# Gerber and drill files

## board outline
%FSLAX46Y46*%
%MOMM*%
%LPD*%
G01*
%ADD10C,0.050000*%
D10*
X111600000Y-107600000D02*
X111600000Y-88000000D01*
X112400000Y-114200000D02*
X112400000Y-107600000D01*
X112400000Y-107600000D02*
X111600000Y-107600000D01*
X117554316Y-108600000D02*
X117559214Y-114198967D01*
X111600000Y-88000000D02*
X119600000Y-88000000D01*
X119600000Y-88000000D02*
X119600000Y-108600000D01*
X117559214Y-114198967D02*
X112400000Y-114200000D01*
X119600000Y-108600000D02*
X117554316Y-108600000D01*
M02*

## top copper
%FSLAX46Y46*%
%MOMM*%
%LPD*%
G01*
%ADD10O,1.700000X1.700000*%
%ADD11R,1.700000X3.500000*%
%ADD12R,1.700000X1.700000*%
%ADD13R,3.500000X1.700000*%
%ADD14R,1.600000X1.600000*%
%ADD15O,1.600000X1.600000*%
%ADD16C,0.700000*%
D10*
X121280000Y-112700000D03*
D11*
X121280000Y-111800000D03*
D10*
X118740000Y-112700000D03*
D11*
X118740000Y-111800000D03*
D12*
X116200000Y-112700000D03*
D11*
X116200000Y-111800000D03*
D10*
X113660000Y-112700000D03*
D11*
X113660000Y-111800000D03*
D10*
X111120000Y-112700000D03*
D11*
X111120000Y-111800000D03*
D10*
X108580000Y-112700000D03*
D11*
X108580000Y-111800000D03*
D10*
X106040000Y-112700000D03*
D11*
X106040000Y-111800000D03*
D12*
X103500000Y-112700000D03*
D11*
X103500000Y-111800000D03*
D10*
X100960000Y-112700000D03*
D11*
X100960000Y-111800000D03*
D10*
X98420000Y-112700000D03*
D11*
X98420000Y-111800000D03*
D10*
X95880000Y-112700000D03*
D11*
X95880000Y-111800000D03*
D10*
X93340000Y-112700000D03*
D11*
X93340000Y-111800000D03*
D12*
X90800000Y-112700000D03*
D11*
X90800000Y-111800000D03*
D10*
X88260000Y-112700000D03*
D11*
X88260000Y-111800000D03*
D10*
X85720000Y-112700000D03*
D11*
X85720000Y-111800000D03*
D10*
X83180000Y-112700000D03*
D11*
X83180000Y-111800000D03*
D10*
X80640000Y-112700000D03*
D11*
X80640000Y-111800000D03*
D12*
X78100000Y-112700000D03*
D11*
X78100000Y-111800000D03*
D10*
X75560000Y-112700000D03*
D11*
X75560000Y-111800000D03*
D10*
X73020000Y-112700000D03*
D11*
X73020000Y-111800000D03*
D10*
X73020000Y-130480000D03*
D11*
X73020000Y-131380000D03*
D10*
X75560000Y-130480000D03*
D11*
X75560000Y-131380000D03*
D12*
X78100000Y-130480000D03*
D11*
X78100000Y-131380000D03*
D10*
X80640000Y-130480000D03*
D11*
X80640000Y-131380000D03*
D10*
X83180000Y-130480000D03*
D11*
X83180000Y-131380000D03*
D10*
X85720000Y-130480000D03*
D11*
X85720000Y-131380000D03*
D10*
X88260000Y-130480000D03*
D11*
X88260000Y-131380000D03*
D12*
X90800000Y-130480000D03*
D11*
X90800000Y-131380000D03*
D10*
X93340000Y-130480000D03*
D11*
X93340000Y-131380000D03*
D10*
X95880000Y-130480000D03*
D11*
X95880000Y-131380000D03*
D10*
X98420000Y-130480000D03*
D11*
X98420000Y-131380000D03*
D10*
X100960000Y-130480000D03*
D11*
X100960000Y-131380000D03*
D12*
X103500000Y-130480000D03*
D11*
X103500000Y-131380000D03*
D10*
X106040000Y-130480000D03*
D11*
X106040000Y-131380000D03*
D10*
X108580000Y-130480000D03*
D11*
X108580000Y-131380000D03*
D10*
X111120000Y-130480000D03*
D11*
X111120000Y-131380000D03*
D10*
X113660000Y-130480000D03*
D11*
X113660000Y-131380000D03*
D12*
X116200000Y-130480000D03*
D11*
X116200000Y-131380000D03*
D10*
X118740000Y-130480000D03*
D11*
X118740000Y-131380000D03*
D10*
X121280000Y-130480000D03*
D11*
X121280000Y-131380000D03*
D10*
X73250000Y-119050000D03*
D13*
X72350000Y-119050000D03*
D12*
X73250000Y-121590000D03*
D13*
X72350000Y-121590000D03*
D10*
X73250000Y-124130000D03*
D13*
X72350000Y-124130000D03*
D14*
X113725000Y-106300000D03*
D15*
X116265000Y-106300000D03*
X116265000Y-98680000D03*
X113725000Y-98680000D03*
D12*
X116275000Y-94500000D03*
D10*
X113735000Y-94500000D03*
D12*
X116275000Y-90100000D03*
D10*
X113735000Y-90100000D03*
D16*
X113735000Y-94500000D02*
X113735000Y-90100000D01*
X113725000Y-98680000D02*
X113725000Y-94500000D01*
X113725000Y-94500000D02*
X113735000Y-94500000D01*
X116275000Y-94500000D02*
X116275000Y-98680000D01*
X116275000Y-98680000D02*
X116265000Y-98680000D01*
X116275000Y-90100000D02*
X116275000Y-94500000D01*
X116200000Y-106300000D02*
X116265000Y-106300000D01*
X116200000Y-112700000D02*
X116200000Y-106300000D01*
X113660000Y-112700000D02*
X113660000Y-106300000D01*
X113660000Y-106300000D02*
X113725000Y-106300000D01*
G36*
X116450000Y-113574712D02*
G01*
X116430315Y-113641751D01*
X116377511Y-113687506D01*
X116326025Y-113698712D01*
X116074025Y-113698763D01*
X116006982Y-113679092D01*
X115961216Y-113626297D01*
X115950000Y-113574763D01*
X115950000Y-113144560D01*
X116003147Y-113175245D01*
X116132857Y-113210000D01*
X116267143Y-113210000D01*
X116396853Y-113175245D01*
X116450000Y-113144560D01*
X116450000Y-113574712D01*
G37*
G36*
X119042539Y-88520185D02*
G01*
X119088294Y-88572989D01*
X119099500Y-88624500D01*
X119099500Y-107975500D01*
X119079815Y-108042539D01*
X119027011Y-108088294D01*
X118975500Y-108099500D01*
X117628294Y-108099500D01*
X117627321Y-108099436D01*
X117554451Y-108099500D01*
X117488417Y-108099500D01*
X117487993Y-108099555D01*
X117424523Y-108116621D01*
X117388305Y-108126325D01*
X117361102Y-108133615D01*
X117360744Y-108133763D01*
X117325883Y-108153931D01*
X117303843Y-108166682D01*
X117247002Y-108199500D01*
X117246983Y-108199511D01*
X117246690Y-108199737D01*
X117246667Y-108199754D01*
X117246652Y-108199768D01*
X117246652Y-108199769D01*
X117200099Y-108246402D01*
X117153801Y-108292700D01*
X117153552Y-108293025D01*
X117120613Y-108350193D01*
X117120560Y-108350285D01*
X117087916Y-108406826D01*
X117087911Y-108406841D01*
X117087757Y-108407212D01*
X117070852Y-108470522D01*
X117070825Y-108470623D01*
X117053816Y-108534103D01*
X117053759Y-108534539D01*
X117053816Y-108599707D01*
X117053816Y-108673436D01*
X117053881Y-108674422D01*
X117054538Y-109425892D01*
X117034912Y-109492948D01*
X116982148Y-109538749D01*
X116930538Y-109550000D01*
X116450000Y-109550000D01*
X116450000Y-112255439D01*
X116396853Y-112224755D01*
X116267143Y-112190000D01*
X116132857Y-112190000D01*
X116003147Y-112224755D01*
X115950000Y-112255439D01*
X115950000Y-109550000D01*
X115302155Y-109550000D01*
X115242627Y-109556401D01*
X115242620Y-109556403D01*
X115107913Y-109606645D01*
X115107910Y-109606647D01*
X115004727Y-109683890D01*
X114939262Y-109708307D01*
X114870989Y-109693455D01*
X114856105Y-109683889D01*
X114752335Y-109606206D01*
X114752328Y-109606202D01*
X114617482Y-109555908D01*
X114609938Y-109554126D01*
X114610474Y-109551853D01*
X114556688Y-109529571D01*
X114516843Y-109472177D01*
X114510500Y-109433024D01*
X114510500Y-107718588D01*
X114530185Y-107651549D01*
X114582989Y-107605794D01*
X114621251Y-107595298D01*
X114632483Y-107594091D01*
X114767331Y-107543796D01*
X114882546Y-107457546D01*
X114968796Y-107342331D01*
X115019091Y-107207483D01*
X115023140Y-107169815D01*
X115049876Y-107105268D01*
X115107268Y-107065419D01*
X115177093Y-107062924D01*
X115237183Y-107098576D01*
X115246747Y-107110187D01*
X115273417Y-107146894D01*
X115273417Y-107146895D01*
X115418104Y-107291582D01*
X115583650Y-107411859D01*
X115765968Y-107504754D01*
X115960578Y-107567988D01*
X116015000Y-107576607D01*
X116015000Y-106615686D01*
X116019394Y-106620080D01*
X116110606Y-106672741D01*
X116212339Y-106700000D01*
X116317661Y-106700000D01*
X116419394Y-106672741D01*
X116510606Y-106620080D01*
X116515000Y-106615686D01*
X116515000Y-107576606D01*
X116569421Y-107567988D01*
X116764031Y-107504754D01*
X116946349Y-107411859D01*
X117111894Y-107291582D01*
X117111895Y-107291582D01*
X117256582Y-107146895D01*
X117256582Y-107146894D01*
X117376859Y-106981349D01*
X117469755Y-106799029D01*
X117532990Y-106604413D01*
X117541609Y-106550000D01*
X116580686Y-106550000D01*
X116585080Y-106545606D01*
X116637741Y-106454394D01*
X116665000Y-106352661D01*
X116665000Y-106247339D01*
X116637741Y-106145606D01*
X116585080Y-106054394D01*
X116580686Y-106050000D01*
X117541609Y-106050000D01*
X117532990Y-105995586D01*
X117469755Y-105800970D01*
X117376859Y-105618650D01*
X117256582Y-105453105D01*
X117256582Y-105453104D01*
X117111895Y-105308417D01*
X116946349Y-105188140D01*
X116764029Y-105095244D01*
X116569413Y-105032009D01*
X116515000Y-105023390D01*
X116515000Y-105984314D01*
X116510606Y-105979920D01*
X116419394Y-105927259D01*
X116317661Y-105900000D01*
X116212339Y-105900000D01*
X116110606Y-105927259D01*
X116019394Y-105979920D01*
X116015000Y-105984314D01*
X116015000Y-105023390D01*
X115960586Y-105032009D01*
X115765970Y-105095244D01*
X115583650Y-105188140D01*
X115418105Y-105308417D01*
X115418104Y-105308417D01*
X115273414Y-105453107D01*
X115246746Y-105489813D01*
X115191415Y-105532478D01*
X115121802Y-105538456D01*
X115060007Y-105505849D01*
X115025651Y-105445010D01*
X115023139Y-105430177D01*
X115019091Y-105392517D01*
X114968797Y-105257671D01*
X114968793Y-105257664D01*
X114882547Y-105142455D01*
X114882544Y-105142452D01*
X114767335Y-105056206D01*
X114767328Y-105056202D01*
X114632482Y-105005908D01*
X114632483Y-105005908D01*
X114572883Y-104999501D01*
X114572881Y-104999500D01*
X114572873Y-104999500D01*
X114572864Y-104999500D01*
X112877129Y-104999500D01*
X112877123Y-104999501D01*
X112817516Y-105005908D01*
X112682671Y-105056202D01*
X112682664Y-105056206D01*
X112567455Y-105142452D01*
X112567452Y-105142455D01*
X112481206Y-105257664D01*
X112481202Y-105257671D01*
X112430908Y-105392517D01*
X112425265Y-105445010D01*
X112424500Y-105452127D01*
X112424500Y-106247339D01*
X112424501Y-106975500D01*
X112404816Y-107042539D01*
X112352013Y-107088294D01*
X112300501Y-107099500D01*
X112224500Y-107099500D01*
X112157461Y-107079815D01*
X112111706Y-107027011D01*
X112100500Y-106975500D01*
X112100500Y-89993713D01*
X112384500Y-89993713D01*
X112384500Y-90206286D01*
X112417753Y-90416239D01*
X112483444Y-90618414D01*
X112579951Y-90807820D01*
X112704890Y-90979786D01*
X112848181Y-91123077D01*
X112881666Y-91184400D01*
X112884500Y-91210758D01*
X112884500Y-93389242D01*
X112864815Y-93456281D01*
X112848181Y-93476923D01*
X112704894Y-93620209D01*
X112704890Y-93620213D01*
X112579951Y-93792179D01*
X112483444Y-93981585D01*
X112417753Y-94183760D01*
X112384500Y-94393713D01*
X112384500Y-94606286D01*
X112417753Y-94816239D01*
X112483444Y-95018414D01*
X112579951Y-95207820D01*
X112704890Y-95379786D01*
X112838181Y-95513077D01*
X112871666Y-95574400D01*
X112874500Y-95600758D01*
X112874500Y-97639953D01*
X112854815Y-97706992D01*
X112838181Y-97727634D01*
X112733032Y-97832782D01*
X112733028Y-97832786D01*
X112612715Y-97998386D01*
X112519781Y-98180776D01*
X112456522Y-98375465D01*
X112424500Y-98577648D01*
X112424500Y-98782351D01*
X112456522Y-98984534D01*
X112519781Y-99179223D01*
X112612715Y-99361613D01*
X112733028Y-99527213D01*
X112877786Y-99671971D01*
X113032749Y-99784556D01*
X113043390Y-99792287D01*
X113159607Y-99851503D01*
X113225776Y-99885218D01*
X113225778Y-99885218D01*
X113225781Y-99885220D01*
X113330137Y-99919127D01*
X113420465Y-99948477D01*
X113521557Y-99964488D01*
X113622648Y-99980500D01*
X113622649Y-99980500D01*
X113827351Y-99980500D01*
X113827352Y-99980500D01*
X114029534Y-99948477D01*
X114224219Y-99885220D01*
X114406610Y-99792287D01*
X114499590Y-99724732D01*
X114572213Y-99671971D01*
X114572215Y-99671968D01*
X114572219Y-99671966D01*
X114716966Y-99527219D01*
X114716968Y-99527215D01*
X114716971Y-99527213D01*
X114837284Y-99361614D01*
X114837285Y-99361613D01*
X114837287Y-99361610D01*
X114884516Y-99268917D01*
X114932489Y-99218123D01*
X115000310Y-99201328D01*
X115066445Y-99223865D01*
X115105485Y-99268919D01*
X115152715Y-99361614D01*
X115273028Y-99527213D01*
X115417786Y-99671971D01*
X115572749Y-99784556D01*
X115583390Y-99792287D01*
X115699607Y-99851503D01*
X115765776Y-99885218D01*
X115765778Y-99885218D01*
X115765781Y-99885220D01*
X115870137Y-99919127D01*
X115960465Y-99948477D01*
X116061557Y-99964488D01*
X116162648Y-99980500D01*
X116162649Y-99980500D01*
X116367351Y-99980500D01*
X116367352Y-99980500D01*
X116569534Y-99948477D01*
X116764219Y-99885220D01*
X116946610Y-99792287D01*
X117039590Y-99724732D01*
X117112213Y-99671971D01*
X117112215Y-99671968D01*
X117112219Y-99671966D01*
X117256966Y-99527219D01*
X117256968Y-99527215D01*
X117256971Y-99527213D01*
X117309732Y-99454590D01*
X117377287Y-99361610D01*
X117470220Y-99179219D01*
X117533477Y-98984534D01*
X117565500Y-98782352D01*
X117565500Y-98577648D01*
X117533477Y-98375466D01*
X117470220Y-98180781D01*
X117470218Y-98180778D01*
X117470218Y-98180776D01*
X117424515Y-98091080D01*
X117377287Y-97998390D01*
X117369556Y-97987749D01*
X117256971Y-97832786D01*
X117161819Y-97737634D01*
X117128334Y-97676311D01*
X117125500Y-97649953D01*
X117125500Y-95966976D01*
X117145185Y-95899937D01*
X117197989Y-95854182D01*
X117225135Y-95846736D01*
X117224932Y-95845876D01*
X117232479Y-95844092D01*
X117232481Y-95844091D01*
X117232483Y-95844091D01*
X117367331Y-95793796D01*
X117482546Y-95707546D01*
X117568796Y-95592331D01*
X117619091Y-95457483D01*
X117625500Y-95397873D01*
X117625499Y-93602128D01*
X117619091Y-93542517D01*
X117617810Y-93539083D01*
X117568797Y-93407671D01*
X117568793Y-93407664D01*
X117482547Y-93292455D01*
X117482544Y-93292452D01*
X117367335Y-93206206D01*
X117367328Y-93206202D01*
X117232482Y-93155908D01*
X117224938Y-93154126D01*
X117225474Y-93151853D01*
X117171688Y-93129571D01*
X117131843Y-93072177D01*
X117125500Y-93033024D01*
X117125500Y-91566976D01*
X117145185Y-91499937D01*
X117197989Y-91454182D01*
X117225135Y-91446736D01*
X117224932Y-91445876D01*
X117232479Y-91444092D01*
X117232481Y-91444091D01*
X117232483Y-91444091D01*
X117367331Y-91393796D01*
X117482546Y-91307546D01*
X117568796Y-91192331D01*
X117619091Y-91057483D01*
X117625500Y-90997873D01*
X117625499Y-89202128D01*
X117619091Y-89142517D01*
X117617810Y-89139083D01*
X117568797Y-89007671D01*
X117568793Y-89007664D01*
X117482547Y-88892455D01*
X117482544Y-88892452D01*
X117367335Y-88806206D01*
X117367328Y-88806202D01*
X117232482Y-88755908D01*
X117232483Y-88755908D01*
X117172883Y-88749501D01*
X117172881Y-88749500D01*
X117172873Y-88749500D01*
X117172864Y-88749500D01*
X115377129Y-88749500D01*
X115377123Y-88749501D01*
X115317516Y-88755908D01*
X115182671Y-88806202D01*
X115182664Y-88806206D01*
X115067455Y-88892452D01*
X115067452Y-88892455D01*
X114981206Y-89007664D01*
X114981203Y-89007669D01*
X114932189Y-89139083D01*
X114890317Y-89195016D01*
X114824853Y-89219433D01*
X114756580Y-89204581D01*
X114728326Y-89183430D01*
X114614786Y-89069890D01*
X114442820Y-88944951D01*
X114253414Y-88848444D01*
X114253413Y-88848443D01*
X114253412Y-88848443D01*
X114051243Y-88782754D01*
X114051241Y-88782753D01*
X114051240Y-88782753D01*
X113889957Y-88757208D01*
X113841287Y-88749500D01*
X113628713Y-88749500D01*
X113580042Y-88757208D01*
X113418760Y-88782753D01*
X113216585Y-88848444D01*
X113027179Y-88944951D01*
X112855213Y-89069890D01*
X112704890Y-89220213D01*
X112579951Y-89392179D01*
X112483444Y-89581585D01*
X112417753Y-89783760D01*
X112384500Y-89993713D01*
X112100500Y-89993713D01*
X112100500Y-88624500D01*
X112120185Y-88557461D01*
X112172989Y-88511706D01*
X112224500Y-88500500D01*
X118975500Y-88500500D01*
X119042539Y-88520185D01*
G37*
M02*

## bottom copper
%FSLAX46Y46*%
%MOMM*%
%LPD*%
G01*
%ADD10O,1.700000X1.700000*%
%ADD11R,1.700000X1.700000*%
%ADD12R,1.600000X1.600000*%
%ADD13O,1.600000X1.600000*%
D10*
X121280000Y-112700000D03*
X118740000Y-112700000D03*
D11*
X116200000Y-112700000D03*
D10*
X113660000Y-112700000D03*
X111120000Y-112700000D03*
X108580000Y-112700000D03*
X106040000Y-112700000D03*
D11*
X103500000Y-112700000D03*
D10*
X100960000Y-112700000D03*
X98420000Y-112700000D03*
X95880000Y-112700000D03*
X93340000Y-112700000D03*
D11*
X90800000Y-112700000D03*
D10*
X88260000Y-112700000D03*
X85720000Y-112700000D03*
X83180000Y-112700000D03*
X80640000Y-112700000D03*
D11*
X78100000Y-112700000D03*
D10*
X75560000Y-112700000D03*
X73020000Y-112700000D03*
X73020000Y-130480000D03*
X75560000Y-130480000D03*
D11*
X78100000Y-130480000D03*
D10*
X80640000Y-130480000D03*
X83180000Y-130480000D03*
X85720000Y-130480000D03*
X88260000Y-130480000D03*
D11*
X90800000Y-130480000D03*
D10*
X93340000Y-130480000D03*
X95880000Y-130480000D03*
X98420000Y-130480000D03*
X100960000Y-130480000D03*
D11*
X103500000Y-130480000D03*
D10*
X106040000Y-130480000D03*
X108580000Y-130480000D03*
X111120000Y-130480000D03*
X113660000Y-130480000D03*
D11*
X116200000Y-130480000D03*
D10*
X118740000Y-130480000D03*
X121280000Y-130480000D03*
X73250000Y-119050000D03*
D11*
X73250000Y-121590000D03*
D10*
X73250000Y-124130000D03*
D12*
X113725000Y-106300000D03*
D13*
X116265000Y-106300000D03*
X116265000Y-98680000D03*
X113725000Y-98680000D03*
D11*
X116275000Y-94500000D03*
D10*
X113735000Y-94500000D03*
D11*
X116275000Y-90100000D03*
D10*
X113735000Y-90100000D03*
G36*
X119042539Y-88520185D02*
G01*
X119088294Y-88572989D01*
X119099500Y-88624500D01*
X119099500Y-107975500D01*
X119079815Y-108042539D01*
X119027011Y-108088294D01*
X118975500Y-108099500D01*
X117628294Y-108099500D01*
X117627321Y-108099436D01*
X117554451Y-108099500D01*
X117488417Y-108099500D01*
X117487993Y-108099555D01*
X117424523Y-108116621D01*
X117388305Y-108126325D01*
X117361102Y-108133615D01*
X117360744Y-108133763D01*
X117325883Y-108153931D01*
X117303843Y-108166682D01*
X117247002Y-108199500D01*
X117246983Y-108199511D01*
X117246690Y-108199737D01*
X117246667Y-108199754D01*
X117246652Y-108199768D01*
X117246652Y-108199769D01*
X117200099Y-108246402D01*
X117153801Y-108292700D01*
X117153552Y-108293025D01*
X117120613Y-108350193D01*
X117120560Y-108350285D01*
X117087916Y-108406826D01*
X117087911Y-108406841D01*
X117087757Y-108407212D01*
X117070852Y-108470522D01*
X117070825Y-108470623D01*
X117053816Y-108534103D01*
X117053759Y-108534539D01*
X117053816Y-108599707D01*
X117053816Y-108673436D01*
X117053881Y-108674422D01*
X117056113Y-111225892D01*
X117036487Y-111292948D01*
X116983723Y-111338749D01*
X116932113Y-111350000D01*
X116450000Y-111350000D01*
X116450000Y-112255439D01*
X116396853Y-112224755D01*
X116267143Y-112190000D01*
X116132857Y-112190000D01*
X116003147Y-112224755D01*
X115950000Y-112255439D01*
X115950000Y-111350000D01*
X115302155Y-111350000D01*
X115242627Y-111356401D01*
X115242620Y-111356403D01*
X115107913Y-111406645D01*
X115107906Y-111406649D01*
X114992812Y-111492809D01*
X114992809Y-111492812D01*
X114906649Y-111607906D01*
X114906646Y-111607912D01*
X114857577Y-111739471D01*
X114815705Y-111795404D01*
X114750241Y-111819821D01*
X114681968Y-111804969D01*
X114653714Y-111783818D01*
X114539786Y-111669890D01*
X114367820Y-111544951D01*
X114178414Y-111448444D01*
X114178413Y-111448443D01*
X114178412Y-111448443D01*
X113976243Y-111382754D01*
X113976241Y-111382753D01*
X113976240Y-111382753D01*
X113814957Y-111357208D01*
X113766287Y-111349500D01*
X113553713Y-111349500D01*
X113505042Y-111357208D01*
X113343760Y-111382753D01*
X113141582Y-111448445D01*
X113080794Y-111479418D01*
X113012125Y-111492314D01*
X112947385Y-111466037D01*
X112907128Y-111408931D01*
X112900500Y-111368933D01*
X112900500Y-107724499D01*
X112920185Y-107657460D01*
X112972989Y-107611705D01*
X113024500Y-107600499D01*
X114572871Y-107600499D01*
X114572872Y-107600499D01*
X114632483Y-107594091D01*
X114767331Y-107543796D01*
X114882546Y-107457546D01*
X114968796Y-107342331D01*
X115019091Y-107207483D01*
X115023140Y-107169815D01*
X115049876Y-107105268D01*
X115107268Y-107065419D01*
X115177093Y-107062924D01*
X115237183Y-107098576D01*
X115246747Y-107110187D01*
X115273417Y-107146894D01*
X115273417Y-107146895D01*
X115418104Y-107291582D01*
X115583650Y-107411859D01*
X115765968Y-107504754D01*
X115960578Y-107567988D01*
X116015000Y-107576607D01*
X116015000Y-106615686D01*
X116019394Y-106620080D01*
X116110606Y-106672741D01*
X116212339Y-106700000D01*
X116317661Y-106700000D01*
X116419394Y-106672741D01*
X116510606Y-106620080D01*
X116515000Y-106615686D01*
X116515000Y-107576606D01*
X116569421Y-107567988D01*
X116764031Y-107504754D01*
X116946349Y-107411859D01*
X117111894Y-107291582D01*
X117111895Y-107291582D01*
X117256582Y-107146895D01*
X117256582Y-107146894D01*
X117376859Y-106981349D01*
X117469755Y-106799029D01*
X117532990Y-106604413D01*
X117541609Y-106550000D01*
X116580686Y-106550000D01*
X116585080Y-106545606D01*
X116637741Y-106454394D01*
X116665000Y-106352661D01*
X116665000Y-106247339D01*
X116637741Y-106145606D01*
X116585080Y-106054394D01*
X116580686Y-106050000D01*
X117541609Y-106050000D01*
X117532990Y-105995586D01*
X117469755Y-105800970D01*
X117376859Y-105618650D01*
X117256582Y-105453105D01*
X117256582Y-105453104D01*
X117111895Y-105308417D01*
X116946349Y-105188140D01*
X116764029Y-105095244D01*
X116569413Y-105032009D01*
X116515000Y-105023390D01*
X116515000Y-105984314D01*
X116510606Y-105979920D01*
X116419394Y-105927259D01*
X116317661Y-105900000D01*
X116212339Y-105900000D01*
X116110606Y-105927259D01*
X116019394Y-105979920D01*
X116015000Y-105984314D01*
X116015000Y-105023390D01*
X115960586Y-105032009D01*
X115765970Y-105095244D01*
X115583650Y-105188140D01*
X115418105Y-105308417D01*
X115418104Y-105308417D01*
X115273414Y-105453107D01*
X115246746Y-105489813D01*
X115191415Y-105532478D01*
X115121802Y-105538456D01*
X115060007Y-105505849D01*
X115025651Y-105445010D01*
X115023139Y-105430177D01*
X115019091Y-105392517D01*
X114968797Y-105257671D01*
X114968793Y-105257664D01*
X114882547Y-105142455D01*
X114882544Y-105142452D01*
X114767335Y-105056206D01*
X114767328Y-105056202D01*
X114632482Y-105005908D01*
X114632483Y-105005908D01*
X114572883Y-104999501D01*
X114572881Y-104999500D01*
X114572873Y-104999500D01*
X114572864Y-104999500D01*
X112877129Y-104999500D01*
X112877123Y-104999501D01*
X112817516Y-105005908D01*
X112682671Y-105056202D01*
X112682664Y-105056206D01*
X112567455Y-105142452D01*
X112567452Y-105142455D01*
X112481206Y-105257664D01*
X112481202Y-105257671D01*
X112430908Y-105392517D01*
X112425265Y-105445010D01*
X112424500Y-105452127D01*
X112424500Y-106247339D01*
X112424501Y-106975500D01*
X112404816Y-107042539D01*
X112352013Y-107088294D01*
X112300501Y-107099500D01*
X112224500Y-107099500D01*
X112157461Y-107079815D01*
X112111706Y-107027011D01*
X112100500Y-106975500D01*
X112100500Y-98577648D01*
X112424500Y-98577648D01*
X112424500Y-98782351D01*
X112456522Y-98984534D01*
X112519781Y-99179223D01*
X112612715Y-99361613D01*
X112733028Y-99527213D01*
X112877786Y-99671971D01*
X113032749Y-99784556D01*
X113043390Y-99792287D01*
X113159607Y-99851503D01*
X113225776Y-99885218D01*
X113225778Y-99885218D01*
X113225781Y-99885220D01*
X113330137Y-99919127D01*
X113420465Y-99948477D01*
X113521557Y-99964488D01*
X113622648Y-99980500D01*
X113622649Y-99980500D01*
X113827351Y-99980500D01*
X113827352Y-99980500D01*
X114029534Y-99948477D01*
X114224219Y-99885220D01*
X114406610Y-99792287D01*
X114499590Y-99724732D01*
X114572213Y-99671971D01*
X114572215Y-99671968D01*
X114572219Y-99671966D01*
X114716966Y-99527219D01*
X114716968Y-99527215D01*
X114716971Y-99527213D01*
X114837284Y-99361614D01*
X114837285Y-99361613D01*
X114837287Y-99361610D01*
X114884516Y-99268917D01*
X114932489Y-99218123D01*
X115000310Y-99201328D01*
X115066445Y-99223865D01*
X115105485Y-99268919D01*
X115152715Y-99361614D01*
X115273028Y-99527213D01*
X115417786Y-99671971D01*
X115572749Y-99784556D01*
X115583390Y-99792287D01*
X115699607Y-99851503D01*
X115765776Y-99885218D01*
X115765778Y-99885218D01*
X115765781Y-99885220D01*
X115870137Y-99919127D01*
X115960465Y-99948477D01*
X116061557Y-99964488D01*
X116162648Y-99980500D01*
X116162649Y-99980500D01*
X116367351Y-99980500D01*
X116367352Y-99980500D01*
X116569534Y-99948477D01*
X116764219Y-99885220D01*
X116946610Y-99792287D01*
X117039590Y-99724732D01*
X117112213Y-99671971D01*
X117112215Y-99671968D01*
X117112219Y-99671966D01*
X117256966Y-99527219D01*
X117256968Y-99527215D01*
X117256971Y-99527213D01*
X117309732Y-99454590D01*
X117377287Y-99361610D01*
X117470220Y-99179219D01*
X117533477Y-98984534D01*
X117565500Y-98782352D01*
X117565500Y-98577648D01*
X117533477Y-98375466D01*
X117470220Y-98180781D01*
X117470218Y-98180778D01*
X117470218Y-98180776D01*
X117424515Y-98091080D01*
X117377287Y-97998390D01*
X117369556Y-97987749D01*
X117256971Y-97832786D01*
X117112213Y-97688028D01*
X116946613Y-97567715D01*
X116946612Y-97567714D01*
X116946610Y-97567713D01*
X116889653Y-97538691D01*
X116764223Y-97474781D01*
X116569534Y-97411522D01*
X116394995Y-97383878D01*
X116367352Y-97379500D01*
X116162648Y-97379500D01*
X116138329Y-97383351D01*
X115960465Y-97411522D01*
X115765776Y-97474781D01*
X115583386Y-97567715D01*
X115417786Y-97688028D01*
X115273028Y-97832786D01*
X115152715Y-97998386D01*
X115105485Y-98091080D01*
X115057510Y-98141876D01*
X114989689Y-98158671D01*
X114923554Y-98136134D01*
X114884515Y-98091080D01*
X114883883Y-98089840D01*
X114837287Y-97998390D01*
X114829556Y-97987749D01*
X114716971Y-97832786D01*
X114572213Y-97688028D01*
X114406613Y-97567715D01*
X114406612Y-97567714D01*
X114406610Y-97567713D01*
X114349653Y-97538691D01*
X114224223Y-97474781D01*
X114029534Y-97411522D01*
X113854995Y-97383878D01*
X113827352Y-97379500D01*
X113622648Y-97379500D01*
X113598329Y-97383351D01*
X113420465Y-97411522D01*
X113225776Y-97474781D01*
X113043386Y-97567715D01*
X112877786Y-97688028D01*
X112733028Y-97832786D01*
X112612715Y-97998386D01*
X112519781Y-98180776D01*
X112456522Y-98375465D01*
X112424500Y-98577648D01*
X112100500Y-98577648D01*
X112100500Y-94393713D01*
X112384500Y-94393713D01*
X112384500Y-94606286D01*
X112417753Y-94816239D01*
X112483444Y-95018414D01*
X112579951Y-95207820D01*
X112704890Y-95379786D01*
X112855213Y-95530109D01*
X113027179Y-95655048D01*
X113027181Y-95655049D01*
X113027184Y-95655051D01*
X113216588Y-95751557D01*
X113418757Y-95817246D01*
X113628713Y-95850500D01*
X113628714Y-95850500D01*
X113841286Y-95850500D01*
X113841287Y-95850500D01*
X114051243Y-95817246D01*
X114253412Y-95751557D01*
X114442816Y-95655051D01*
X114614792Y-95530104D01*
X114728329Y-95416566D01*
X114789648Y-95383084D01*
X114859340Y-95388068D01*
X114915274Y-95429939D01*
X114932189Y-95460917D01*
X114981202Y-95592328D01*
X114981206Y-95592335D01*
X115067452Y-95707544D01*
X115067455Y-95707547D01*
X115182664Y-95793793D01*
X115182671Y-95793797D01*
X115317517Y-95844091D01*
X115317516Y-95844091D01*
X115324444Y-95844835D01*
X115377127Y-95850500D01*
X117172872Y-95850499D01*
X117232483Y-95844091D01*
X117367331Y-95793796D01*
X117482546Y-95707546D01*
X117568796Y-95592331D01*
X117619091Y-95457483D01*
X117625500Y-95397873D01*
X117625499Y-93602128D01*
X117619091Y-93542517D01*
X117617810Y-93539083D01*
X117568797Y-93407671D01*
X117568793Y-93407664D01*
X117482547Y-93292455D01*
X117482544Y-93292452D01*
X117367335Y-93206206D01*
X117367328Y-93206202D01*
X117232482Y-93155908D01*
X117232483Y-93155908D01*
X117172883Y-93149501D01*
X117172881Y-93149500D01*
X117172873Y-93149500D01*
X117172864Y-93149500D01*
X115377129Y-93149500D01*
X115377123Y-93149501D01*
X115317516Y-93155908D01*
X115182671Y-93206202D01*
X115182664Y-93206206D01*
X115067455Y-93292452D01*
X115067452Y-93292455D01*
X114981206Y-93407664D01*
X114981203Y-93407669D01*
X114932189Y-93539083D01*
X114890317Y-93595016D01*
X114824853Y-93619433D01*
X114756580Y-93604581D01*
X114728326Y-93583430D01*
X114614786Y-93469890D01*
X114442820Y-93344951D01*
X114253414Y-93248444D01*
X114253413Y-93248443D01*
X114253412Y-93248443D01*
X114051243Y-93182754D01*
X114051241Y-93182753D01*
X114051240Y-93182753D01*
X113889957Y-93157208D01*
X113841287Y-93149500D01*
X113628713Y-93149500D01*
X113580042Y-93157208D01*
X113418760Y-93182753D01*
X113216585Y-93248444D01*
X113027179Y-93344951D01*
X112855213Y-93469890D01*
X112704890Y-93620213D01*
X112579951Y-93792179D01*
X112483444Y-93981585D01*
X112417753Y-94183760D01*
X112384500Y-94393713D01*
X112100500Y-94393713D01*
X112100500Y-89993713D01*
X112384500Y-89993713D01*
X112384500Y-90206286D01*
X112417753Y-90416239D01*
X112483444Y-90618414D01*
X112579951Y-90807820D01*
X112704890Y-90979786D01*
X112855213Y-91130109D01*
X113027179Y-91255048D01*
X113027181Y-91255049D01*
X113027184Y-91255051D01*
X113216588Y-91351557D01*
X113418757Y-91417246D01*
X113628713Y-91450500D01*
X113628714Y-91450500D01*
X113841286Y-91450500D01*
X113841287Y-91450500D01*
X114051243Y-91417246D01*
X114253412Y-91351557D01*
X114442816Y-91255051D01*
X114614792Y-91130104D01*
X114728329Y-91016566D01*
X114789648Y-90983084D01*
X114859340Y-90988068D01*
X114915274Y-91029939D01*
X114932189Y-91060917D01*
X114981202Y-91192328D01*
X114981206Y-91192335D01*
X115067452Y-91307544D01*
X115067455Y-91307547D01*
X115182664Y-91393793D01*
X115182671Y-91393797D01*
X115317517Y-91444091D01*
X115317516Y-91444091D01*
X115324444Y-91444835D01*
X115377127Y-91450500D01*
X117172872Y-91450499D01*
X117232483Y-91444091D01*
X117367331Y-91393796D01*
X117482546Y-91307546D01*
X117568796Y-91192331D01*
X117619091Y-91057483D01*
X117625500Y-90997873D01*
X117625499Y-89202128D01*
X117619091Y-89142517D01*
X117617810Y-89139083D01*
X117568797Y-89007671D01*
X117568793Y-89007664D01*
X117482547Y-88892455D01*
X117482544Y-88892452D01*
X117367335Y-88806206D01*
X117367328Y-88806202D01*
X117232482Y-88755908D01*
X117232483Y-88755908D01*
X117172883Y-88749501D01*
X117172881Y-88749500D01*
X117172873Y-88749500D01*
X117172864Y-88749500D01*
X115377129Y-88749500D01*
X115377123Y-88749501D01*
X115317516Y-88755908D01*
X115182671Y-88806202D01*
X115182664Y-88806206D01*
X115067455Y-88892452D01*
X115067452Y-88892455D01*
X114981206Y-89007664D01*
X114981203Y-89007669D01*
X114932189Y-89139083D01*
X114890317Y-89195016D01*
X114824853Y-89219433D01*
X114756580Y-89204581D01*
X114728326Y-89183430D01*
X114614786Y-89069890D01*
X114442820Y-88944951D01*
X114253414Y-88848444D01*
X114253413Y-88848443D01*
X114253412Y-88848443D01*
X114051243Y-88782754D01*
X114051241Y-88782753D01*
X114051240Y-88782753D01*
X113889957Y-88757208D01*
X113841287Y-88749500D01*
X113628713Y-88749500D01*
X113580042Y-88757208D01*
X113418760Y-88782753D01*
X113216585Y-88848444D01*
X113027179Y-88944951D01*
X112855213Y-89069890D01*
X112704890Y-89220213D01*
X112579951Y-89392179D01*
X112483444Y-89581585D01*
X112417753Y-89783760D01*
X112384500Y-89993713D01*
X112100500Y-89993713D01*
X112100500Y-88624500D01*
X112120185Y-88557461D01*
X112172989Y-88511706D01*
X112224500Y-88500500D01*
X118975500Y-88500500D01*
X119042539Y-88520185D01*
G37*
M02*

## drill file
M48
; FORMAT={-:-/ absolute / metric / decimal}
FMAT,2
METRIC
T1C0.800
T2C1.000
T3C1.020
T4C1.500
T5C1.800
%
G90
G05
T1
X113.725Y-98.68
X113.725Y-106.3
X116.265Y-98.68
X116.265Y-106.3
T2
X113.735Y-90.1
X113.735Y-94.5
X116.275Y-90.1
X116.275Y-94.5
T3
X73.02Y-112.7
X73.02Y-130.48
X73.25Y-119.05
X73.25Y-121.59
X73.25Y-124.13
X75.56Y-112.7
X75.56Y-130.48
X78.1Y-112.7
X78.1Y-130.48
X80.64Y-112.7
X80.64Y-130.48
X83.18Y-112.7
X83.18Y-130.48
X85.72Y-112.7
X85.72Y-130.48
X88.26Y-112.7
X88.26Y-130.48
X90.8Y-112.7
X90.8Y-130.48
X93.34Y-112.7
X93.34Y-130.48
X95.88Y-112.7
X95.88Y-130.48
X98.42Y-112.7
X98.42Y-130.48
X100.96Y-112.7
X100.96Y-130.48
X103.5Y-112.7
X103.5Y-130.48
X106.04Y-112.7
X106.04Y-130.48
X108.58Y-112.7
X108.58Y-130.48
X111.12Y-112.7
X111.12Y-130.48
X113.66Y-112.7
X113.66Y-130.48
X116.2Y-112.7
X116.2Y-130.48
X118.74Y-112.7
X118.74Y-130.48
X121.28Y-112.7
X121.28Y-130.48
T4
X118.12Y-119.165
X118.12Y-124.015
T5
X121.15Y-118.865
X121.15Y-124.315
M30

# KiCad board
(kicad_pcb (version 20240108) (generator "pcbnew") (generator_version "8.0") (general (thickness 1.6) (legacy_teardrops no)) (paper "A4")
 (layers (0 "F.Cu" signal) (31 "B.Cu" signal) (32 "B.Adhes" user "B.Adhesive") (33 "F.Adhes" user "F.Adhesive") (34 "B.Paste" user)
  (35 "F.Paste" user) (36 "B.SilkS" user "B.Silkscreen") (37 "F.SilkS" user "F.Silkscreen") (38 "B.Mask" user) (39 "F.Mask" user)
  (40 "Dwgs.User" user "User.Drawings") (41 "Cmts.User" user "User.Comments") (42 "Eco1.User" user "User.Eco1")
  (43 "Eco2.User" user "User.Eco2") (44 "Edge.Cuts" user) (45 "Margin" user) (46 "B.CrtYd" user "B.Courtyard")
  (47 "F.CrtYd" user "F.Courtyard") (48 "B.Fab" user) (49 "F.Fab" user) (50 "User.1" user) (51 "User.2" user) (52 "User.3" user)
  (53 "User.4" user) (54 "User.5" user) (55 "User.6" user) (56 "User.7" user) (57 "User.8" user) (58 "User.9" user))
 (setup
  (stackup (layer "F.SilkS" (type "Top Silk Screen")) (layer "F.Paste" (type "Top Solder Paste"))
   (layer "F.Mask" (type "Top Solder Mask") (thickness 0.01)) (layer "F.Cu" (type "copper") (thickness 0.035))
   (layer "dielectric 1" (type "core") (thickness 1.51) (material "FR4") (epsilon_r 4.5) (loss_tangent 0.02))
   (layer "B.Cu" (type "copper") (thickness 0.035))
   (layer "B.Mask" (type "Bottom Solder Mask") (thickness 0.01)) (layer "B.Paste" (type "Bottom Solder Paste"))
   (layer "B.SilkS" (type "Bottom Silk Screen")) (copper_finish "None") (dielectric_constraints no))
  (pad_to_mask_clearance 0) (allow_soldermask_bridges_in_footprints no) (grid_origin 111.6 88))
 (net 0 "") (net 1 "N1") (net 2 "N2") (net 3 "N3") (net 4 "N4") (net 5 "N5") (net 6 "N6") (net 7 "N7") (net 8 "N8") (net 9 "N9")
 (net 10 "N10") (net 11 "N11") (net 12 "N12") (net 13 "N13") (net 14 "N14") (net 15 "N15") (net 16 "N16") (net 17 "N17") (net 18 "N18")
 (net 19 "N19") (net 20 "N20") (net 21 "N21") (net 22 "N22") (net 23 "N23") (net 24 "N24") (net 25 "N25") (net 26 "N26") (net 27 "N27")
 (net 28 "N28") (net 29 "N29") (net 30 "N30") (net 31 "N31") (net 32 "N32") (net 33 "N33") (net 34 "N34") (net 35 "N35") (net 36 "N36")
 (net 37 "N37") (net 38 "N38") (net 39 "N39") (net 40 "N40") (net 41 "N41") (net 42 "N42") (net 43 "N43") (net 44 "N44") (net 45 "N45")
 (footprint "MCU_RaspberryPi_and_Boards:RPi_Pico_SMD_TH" (layer "F.Cu") (at 97.15 121.59 -90)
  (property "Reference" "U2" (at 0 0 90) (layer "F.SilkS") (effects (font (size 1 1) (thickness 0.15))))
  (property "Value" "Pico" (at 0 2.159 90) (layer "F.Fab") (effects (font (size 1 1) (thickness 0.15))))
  (pad "" np_thru_hole oval (at -2.725 -24 270) (size 1.8 1.8) (drill 1.8) (layers "*.Cu" "*.Mask"))
  (pad "" np_thru_hole oval (at -2.425 -20.97 270) (size 1.5 1.5) (drill 1.5) (layers "*.Cu" "*.Mask"))
  (pad "" np_thru_hole oval (at 2.425 -20.97 270) (size 1.5 1.5) (drill 1.5) (layers "*.Cu" "*.Mask"))
  (pad "" np_thru_hole oval (at 2.725 -24 270) (size 1.8 1.8) (drill 1.8) (layers "*.Cu" "*.Mask"))
  (pad "1" thru_hole oval (at -8.89 -24.13 270) (size 1.7 1.7) (drill 1.02) (layers "*.Cu" "*.Mask") (remove_unused_layers no) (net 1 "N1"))
  (pad "1" smd rect (at -8.89 -24.13 270) (size 3.5 1.7) (drill (offset -0.9 0)) (layers "F.Cu" "F.Mask") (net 1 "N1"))
  (pad "2" thru_hole oval (at -8.89 -21.59 270) (size 1.7 1.7) (drill 1.02) (layers "*.Cu" "*.Mask") (remove_unused_layers no) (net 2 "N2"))
  (pad "2" smd rect (at -8.89 -21.59 270) (size 3.5 1.7) (drill (offset -0.9 0)) (layers "F.Cu" "F.Mask") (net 2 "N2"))
  (pad "3" thru_hole rect (at -8.89 -19.05 270) (size 1.7 1.7) (drill 1.02) (layers "*.Cu" "*.Mask") (remove_unused_layers no) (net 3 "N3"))
  (pad "3" smd rect (at -8.89 -19.05 270) (size 3.5 1.7) (drill (offset -0.9 0)) (layers "F.Cu" "F.Mask") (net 3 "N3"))
  (pad "4" thru_hole oval (at -8.89 -16.51 270) (size 1.7 1.7) (drill 1.02) (layers "*.Cu" "*.Mask") (remove_unused_layers no) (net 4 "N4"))
  (pad "4" smd rect (at -8.89 -16.51 270) (size 3.5 1.7) (drill (offset -0.9 0)) (layers "F.Cu" "F.Mask") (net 4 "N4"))
  (pad "5" thru_hole oval (at -8.89 -13.97 270) (size 1.7 1.7) (drill 1.02) (layers "*.Cu" "*.Mask") (remove_unused_layers no) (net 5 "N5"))
  (pad "5" smd rect (at -8.89 -13.97 270) (size 3.5 1.7) (drill (offset -0.9 0)) (layers "F.Cu" "F.Mask") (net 5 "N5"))
  (pad "6" thru_hole oval (at -8.89 -11.43 270) (size 1.7 1.7) (drill 1.02) (layers "*.Cu" "*.Mask") (remove_unused_layers no) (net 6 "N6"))
  (pad "6" smd rect (at -8.89 -11.43 270) (size 3.5 1.7) (drill (offset -0.9 0)) (layers "F.Cu" "F.Mask") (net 6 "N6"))
  (pad "7" thru_hole oval (at -8.89 -8.89 270) (size 1.7 1.7) (drill 1.02) (layers "*.Cu" "*.Mask") (remove_unused_layers no) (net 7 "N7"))
  (pad "7" smd rect (at -8.89 -8.89 270) (size 3.5 1.7) (drill (offset -0.9 0)) (layers "F.Cu" "F.Mask") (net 7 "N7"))
  (pad "8" thru_hole rect (at -8.89 -6.35 270) (size 1.7 1.7) (drill 1.02) (layers "*.Cu" "*.Mask") (remove_unused_layers no) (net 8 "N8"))
  (pad "8" smd rect (at -8.89 -6.35 270) (size 3.5 1.7) (drill (offset -0.9 0)) (layers "F.Cu" "F.Mask") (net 8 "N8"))
  (pad "9" thru_hole oval (at -8.89 -3.81 270) (size 1.7 1.7) (drill 1.02) (layers "*.Cu" "*.Mask") (remove_unused_layers no) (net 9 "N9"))
  (pad "9" smd rect (at -8.89 -3.81 270) (size 3.5 1.7) (drill (offset -0.9 0)) (layers "F.Cu" "F.Mask") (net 9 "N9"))
  (pad "10" thru_hole oval (at -8.89 -1.27 270) (size 1.7 1.7) (drill 1.02) (layers "*.Cu" "*.Mask") (remove_unused_layers no)
   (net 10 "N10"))
  (pad "10" smd rect (at -8.89 -1.27 270) (size 3.5 1.7) (drill (offset -0.9 0)) (layers "F.Cu" "F.Mask") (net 10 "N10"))
  (pad "11" thru_hole oval (at -8.89 1.27 270) (size 1.7 1.7) (drill 1.02) (layers "*.Cu" "*.Mask") (remove_unused_layers no) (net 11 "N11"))
  (pad "11" smd rect (at -8.89 1.27 270) (size 3.5 1.7) (drill (offset -0.9 0)) (layers "F.Cu" "F.Mask") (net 11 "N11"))
  (pad "12" thru_hole oval (at -8.89 3.81 270) (size 1.7 1.7) (drill 1.02) (layers "*.Cu" "*.Mask") (remove_unused_layers no) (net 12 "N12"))
  (pad "12" smd rect (at -8.89 3.81 270) (size 3.5 1.7) (drill (offset -0.9 0)) (layers "F.Cu" "F.Mask") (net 12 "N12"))
  (pad "13" thru_hole rect (at -8.89 6.35 270) (size 1.7 1.7) (drill 1.02) (layers "*.Cu" "*.Mask") (remove_unused_layers no) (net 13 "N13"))
  (pad "13" smd rect (at -8.89 6.35 270) (size 3.5 1.7) (drill (offset -0.9 0)) (layers "F.Cu" "F.Mask") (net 13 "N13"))
  (pad "14" thru_hole oval (at -8.89 8.89 270) (size 1.7 1.7) (drill 1.02) (layers "*.Cu" "*.Mask") (remove_unused_layers no) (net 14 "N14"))
  (pad "14" smd rect (at -8.89 8.89 270) (size 3.5 1.7) (drill (offset -0.9 0)) (layers "F.Cu" "F.Mask") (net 14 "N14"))
  (pad "15" thru_hole oval (at -8.89 11.43 270) (size 1.7 1.7) (drill 1.02) (layers "*.Cu" "*.Mask") (remove_unused_layers no)
   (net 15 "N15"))
  (pad "15" smd rect (at -8.89 11.43 270) (size 3.5 1.7) (drill (offset -0.9 0)) (layers "F.Cu" "F.Mask") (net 15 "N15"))
  (pad "16" thru_hole oval (at -8.89 13.97 270) (size 1.7 1.7) (drill 1.02) (layers "*.Cu" "*.Mask") (remove_unused_layers no)
   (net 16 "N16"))
  (pad "16" smd rect (at -8.89 13.97 270) (size 3.5 1.7) (drill (offset -0.9 0)) (layers "F.Cu" "F.Mask") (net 16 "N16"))
  (pad "17" thru_hole oval (at -8.89 16.51 270) (size 1.7 1.7) (drill 1.02) (layers "*.Cu" "*.Mask") (remove_unused_layers no)
   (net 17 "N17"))
  (pad "17" smd rect (at -8.89 16.51 270) (size 3.5 1.7) (drill (offset -0.9 0)) (layers "F.Cu" "F.Mask") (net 17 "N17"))
  (pad "18" thru_hole rect (at -8.89 19.05 270) (size 1.7 1.7) (drill 1.02) (layers "*.Cu" "*.Mask") (remove_unused_layers no)
   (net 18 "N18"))
  (pad "18" smd rect (at -8.89 19.05 270) (size 3.5 1.7) (drill (offset -0.9 0)) (layers "F.Cu" "F.Mask") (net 18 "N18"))
  (pad "19" thru_hole oval (at -8.89 21.59 270) (size 1.7 1.7) (drill 1.02) (layers "*.Cu" "*.Mask") (remove_unused_layers no)
   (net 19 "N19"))
  (pad "19" smd rect (at -8.89 21.59 270) (size 3.5 1.7) (drill (offset -0.9 0)) (layers "F.Cu" "F.Mask") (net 19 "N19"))
  (pad "20" thru_hole oval (at -8.89 24.13 270) (size 1.7 1.7) (drill 1.02) (layers "*.Cu" "*.Mask") (remove_unused_layers no)
   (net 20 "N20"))
  (pad "20" smd rect (at -8.89 24.13 270) (size 3.5 1.7) (drill (offset -0.9 0)) (layers "F.Cu" "F.Mask") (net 20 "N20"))
  (pad "21" thru_hole oval (at 8.89 24.13 270) (size 1.7 1.7) (drill 1.02) (layers "*.Cu" "*.Mask") (remove_unused_layers no) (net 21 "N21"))
  (pad "21" smd rect (at 8.89 24.13 270) (size 3.5 1.7) (drill (offset 0.9 0)) (layers "F.Cu" "F.Mask") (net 21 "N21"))
  (pad "22" thru_hole oval (at 8.89 21.59 270) (size 1.7 1.7) (drill 1.02) (layers "*.Cu" "*.Mask") (remove_unused_layers no) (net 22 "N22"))
  (pad "22" smd rect (at 8.89 21.59 270) (size 3.5 1.7) (drill (offset 0.9 0)) (layers "F.Cu" "F.Mask") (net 22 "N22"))
  (pad "23" thru_hole rect (at 8.89 19.05 270) (size 1.7 1.7) (drill 1.02) (layers "*.Cu" "*.Mask") (remove_unused_layers no) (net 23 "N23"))
  (pad "23" smd rect (at 8.89 19.05 270) (size 3.5 1.7) (drill (offset 0.9 0)) (layers "F.Cu" "F.Mask") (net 23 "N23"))
  (pad "24" thru_hole oval (at 8.89 16.51 270) (size 1.7 1.7) (drill 1.02) (layers "*.Cu" "*.Mask") (remove_unused_layers no) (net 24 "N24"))
  (pad "24" smd rect (at 8.89 16.51 270) (size 3.5 1.7) (drill (offset 0.9 0)) (layers "F.Cu" "F.Mask") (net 24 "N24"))
  (pad "25" thru_hole oval (at 8.89 13.97 270) (size 1.7 1.7) (drill 1.02) (layers "*.Cu" "*.Mask") (remove_unused_layers no) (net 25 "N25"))
  (pad "25" smd rect (at 8.89 13.97 270) (size 3.5 1.7) (drill (offset 0.9 0)) (layers "F.Cu" "F.Mask") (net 25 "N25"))
  (pad "26" thru_hole oval (at 8.89 11.43 270) (size 1.7 1.7) (drill 1.02) (layers "*.Cu" "*.Mask") (remove_unused_layers no) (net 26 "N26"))
  (pad "26" smd rect (at 8.89 11.43 270) (size 3.5 1.7) (drill (offset 0.9 0)) (layers "F.Cu" "F.Mask") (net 26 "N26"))
  (pad "27" thru_hole oval (at 8.89 8.89 270) (size 1.7 1.7) (drill 1.02) (layers "*.Cu" "*.Mask") (remove_unused_layers no) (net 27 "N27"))
  (pad "27" smd rect (at 8.89 8.89 270) (size 3.5 1.7) (drill (offset 0.9 0)) (layers "F.Cu" "F.Mask") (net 27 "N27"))
  (pad "28" thru_hole rect (at 8.89 6.35 270) (size 1.7 1.7) (drill 1.02) (layers "*.Cu" "*.Mask") (remove_unused_layers no) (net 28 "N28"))
  (pad "28" smd rect (at 8.89 6.35 270) (size 3.5 1.7) (drill (offset 0.9 0)) (layers "F.Cu" "F.Mask") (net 28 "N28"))
  (pad "29" thru_hole oval (at 8.89 3.81 270) (size 1.7 1.7) (drill 1.02) (layers "*.Cu" "*.Mask") (remove_unused_layers no) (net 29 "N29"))
  (pad "29" smd rect (at 8.89 3.81 270) (size 3.5 1.7) (drill (offset 0.9 0)) (layers "F.Cu" "F.Mask") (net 29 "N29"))
  (pad "30" thru_hole oval (at 8.89 1.27 270) (size 1.7 1.7) (drill 1.02) (layers "*.Cu" "*.Mask") (remove_unused_layers no) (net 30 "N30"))
  (pad "30" smd rect (at 8.89 1.27 270) (size 3.5 1.7) (drill (offset 0.9 0)) (layers "F.Cu" "F.Mask") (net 30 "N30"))
  (pad "31" thru_hole oval (at 8.89 -1.27 270) (size 1.7 1.7) (drill 1.02) (layers "*.Cu" "*.Mask") (remove_unused_layers no) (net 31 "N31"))
  (pad "31" smd rect (at 8.89 -1.27 270) (size 3.5 1.7) (drill (offset 0.9 0)) (layers "F.Cu" "F.Mask") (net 31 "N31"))
  (pad "32" thru_hole oval (at 8.89 -3.81 270) (size 1.7 1.7) (drill 1.02) (layers "*.Cu" "*.Mask") (remove_unused_layers no) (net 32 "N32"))
  (pad "32" smd rect (at 8.89 -3.81 270) (size 3.5 1.7) (drill (offset 0.9 0)) (layers "F.Cu" "F.Mask") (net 32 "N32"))
  (pad "33" thru_hole rect (at 8.89 -6.35 270) (size 1.7 1.7) (drill 1.02) (layers "*.Cu" "*.Mask") (remove_unused_layers no) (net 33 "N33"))
  (pad "33" smd rect (at 8.89 -6.35 270) (size 3.5 1.7) (drill (offset 0.9 0)) (layers "F.Cu" "F.Mask") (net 33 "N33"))
  (pad "34" thru_hole oval (at 8.89 -8.89 270) (size 1.7 1.7) (drill 1.02) (layers "*.Cu" "*.Mask") (remove_unused_layers no) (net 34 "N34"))
  (pad "34" smd rect (at 8.89 -8.89 270) (size 3.5 1.7) (drill (offset 0.9 0)) (layers "F.Cu" "F.Mask") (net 34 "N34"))
  (pad "35" thru_hole oval (at 8.89 -11.43 270) (size 1.7 1.7) (drill 1.02) (layers "*.Cu" "*.Mask") (remove_unused_layers no)
   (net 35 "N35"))
  (pad "35" smd rect (at 8.89 -11.43 270) (size 3.5 1.7) (drill (offset 0.9 0)) (layers "F.Cu" "F.Mask") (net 35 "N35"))
  (pad "36" thru_hole oval (at 8.89 -13.97 270) (size 1.7 1.7) (drill 1.02) (layers "*.Cu" "*.Mask") (remove_unused_layers no)
   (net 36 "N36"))
  (pad "36" smd rect (at 8.89 -13.97 270) (size 3.5 1.7) (drill (offset 0.9 0)) (layers "F.Cu" "F.Mask") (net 36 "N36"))
  (pad "37" thru_hole oval (at 8.89 -16.51 270) (size 1.7 1.7) (drill 1.02) (layers "*.Cu" "*.Mask") (remove_unused_layers no)
   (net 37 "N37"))
  (pad "37" smd rect (at 8.89 -16.51 270) (size 3.5 1.7) (drill (offset 0.9 0)) (layers "F.Cu" "F.Mask") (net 37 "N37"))
  (pad "38" thru_hole rect (at 8.89 -19.05 270) (size 1.7 1.7) (drill 1.02) (layers "*.Cu" "*.Mask") (remove_unused_layers no)
   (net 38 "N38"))
  (pad "38" smd rect (at 8.89 -19.05 270) (size 3.5 1.7) (drill (offset 0.9 0)) (layers "F.Cu" "F.Mask") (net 38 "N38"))
  (pad "39" thru_hole oval (at 8.89 -21.59 270) (size 1.7 1.7) (drill 1.02) (layers "*.Cu" "*.Mask") (remove_unused_layers no)
   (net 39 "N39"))
  (pad "39" smd rect (at 8.89 -21.59 270) (size 3.5 1.7) (drill (offset 0.9 0)) (layers "F.Cu" "F.Mask") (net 39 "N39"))
  (pad "40" thru_hole oval (at 8.89 -24.13 270) (size 1.7 1.7) (drill 1.02) (layers "*.Cu" "*.Mask") (remove_unused_layers no)
   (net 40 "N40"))
  (pad "40" smd rect (at 8.89 -24.13 270) (size 3.5 1.7) (drill (offset 0.9 0)) (layers "F.Cu" "F.Mask") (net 40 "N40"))
  (pad "41" thru_hole oval (at -2.54 23.9 270) (size 1.7 1.7) (drill 1.02) (layers "*.Cu" "*.Mask") (remove_unused_layers no) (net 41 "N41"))
  (pad "41" smd rect (at -2.54 23.9) (size 3.5 1.7) (drill (offset -0.9 0)) (layers "F.Cu" "F.Mask") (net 41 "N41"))
  (pad "42" thru_hole rect (at 0 23.9 270) (size 1.7 1.7) (drill 1.02) (layers "*.Cu" "*.Mask") (remove_unused_layers no) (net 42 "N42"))
  (pad "42" smd rect (at 0 23.9) (size 3.5 1.7) (drill (offset -0.9 0)) (layers "F.Cu" "F.Mask") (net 42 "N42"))
  (pad "43" thru_hole oval (at 2.54 23.9 270) (size 1.7 1.7) (drill 1.02) (layers "*.Cu" "*.Mask") (remove_unused_layers no) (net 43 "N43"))
  (pad "43" smd rect (at 2.54 23.9) (size 3.5 1.7) (drill (offset -0.9 0)) (layers "F.Cu" "F.Mask") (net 43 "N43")))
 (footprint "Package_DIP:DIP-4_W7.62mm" (layer "F.Cu") (at 113.725 106.3 90)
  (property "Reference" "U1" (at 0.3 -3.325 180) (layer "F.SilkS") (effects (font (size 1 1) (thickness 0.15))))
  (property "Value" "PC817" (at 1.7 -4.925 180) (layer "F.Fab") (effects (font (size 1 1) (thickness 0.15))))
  (pad "1" thru_hole rect (at 0 0 90) (size 1.6 1.6) (drill 0.8) (layers "*.Cu" "*.Mask") (remove_unused_layers no) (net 4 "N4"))
  (pad "2" thru_hole oval (at 0 2.54 90) (size 1.6 1.6) (drill 0.8) (layers "*.Cu" "*.Mask") (remove_unused_layers no) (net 3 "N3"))
  (pad "3" thru_hole oval (at 7.62 2.54 90) (size 1.6 1.6) (drill 0.8) (layers "*.Cu" "*.Mask") (remove_unused_layers no) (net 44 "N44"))
  (pad "4" thru_hole oval (at 7.62 0 90) (size 1.6 1.6) (drill 0.8) (layers "*.Cu" "*.Mask") (remove_unused_layers no) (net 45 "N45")))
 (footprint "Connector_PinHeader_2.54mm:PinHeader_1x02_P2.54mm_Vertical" (layer "F.Cu") (at 116.275 94.5 -90)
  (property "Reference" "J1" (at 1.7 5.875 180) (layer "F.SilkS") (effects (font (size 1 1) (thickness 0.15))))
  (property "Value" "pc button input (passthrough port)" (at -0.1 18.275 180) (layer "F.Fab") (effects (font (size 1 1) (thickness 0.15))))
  (pad "1" thru_hole rect (at 0 0 270) (size 1.7 1.7) (drill 1) (layers "*.Cu" "*.Mask") (remove_unused_layers no) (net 44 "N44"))
  (pad "2" thru_hole oval (at 0 2.54 270) (size 1.7 1.7) (drill 1) (layers "*.Cu" "*.Mask") (remove_unused_layers no) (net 45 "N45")))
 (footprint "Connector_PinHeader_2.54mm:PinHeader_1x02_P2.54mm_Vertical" (layer "F.Cu") (at 116.275 90.1 -90)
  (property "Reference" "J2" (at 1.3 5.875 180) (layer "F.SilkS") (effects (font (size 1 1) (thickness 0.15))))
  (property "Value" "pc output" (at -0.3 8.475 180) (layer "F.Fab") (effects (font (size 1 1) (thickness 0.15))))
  (pad "1" thru_hole rect (at 0 0 270) (size 1.7 1.7) (drill 1) (layers "*.Cu" "*.Mask") (remove_unused_layers no) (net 44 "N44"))
  (pad "2" thru_hole oval (at 0 2.54 270) (size 1.7 1.7) (drill 1) (layers "*.Cu" "*.Mask") (remove_unused_layers no) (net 45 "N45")))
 (gr_line (start 111.6 107.6) (end 111.6 88) (stroke (width 0.05) (type default)) (layer "Edge.Cuts"))
 (gr_line (start 112.4 114.2) (end 112.4 107.6) (stroke (width 0.05) (type default)) (layer "Edge.Cuts"))
 (gr_line (start 112.4 107.6) (end 111.6 107.6) (stroke (width 0.05) (type default)) (layer "Edge.Cuts"))
 (gr_line (start 117.554316 108.6) (end 117.559214 114.198967) (stroke (width 0.05) (type default)) (layer "Edge.Cuts"))
 (gr_line (start 111.6 88) (end 119.6 88) (stroke (width 0.05) (type default)) (layer "Edge.Cuts"))
 (gr_line (start 119.6 88) (end 119.6 108.6) (stroke (width 0.05) (type default)) (layer "Edge.Cuts"))
 (gr_line (start 117.559214 114.198967) (end 112.4 114.2) (stroke (width 0.05) (type default)) (layer "Edge.Cuts"))
 (gr_line (start 119.6 108.6) (end 117.554316 108.6) (stroke (width 0.05) (type default)) (layer "Edge.Cuts"))
 (segment (start 113.735 94.5) (end 113.735 90.1) (width 0.7) (layer "F.Cu") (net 45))
 (segment (start 113.725 98.68) (end 113.725 94.5) (width 0.7) (layer "F.Cu") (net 45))
 (segment (start 113.725 94.5) (end 113.735 94.5) (width 0.7) (layer "F.Cu") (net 45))
 (segment (start 116.275 94.5) (end 116.275 98.68) (width 0.7) (layer "F.Cu") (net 44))
 (segment (start 116.275 98.68) (end 116.265 98.68) (width 0.7) (layer "F.Cu") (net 44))
 (segment (start 116.275 90.1) (end 116.275 94.5) (width 0.7) (layer "F.Cu") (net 44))
 (segment (start 116.2 106.3) (end 116.265 106.3) (width 0.7) (layer "F.Cu") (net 3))
 (segment (start 116.2 112.7) (end 116.2 106.3) (width 0.7) (layer "F.Cu") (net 3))
 (segment (start 113.66 112.7) (end 113.66 106.3) (width 0.7) (layer "F.Cu") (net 4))
 (segment (start 113.66 106.3) (end 113.725 106.3) (width 0.7) (layer "F.Cu") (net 4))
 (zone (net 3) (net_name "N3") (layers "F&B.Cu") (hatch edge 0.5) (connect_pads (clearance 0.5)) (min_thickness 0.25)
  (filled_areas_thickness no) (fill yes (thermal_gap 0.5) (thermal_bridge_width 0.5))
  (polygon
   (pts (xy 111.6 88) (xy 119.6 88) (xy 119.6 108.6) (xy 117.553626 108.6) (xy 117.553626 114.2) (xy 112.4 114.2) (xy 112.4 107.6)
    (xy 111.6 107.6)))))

